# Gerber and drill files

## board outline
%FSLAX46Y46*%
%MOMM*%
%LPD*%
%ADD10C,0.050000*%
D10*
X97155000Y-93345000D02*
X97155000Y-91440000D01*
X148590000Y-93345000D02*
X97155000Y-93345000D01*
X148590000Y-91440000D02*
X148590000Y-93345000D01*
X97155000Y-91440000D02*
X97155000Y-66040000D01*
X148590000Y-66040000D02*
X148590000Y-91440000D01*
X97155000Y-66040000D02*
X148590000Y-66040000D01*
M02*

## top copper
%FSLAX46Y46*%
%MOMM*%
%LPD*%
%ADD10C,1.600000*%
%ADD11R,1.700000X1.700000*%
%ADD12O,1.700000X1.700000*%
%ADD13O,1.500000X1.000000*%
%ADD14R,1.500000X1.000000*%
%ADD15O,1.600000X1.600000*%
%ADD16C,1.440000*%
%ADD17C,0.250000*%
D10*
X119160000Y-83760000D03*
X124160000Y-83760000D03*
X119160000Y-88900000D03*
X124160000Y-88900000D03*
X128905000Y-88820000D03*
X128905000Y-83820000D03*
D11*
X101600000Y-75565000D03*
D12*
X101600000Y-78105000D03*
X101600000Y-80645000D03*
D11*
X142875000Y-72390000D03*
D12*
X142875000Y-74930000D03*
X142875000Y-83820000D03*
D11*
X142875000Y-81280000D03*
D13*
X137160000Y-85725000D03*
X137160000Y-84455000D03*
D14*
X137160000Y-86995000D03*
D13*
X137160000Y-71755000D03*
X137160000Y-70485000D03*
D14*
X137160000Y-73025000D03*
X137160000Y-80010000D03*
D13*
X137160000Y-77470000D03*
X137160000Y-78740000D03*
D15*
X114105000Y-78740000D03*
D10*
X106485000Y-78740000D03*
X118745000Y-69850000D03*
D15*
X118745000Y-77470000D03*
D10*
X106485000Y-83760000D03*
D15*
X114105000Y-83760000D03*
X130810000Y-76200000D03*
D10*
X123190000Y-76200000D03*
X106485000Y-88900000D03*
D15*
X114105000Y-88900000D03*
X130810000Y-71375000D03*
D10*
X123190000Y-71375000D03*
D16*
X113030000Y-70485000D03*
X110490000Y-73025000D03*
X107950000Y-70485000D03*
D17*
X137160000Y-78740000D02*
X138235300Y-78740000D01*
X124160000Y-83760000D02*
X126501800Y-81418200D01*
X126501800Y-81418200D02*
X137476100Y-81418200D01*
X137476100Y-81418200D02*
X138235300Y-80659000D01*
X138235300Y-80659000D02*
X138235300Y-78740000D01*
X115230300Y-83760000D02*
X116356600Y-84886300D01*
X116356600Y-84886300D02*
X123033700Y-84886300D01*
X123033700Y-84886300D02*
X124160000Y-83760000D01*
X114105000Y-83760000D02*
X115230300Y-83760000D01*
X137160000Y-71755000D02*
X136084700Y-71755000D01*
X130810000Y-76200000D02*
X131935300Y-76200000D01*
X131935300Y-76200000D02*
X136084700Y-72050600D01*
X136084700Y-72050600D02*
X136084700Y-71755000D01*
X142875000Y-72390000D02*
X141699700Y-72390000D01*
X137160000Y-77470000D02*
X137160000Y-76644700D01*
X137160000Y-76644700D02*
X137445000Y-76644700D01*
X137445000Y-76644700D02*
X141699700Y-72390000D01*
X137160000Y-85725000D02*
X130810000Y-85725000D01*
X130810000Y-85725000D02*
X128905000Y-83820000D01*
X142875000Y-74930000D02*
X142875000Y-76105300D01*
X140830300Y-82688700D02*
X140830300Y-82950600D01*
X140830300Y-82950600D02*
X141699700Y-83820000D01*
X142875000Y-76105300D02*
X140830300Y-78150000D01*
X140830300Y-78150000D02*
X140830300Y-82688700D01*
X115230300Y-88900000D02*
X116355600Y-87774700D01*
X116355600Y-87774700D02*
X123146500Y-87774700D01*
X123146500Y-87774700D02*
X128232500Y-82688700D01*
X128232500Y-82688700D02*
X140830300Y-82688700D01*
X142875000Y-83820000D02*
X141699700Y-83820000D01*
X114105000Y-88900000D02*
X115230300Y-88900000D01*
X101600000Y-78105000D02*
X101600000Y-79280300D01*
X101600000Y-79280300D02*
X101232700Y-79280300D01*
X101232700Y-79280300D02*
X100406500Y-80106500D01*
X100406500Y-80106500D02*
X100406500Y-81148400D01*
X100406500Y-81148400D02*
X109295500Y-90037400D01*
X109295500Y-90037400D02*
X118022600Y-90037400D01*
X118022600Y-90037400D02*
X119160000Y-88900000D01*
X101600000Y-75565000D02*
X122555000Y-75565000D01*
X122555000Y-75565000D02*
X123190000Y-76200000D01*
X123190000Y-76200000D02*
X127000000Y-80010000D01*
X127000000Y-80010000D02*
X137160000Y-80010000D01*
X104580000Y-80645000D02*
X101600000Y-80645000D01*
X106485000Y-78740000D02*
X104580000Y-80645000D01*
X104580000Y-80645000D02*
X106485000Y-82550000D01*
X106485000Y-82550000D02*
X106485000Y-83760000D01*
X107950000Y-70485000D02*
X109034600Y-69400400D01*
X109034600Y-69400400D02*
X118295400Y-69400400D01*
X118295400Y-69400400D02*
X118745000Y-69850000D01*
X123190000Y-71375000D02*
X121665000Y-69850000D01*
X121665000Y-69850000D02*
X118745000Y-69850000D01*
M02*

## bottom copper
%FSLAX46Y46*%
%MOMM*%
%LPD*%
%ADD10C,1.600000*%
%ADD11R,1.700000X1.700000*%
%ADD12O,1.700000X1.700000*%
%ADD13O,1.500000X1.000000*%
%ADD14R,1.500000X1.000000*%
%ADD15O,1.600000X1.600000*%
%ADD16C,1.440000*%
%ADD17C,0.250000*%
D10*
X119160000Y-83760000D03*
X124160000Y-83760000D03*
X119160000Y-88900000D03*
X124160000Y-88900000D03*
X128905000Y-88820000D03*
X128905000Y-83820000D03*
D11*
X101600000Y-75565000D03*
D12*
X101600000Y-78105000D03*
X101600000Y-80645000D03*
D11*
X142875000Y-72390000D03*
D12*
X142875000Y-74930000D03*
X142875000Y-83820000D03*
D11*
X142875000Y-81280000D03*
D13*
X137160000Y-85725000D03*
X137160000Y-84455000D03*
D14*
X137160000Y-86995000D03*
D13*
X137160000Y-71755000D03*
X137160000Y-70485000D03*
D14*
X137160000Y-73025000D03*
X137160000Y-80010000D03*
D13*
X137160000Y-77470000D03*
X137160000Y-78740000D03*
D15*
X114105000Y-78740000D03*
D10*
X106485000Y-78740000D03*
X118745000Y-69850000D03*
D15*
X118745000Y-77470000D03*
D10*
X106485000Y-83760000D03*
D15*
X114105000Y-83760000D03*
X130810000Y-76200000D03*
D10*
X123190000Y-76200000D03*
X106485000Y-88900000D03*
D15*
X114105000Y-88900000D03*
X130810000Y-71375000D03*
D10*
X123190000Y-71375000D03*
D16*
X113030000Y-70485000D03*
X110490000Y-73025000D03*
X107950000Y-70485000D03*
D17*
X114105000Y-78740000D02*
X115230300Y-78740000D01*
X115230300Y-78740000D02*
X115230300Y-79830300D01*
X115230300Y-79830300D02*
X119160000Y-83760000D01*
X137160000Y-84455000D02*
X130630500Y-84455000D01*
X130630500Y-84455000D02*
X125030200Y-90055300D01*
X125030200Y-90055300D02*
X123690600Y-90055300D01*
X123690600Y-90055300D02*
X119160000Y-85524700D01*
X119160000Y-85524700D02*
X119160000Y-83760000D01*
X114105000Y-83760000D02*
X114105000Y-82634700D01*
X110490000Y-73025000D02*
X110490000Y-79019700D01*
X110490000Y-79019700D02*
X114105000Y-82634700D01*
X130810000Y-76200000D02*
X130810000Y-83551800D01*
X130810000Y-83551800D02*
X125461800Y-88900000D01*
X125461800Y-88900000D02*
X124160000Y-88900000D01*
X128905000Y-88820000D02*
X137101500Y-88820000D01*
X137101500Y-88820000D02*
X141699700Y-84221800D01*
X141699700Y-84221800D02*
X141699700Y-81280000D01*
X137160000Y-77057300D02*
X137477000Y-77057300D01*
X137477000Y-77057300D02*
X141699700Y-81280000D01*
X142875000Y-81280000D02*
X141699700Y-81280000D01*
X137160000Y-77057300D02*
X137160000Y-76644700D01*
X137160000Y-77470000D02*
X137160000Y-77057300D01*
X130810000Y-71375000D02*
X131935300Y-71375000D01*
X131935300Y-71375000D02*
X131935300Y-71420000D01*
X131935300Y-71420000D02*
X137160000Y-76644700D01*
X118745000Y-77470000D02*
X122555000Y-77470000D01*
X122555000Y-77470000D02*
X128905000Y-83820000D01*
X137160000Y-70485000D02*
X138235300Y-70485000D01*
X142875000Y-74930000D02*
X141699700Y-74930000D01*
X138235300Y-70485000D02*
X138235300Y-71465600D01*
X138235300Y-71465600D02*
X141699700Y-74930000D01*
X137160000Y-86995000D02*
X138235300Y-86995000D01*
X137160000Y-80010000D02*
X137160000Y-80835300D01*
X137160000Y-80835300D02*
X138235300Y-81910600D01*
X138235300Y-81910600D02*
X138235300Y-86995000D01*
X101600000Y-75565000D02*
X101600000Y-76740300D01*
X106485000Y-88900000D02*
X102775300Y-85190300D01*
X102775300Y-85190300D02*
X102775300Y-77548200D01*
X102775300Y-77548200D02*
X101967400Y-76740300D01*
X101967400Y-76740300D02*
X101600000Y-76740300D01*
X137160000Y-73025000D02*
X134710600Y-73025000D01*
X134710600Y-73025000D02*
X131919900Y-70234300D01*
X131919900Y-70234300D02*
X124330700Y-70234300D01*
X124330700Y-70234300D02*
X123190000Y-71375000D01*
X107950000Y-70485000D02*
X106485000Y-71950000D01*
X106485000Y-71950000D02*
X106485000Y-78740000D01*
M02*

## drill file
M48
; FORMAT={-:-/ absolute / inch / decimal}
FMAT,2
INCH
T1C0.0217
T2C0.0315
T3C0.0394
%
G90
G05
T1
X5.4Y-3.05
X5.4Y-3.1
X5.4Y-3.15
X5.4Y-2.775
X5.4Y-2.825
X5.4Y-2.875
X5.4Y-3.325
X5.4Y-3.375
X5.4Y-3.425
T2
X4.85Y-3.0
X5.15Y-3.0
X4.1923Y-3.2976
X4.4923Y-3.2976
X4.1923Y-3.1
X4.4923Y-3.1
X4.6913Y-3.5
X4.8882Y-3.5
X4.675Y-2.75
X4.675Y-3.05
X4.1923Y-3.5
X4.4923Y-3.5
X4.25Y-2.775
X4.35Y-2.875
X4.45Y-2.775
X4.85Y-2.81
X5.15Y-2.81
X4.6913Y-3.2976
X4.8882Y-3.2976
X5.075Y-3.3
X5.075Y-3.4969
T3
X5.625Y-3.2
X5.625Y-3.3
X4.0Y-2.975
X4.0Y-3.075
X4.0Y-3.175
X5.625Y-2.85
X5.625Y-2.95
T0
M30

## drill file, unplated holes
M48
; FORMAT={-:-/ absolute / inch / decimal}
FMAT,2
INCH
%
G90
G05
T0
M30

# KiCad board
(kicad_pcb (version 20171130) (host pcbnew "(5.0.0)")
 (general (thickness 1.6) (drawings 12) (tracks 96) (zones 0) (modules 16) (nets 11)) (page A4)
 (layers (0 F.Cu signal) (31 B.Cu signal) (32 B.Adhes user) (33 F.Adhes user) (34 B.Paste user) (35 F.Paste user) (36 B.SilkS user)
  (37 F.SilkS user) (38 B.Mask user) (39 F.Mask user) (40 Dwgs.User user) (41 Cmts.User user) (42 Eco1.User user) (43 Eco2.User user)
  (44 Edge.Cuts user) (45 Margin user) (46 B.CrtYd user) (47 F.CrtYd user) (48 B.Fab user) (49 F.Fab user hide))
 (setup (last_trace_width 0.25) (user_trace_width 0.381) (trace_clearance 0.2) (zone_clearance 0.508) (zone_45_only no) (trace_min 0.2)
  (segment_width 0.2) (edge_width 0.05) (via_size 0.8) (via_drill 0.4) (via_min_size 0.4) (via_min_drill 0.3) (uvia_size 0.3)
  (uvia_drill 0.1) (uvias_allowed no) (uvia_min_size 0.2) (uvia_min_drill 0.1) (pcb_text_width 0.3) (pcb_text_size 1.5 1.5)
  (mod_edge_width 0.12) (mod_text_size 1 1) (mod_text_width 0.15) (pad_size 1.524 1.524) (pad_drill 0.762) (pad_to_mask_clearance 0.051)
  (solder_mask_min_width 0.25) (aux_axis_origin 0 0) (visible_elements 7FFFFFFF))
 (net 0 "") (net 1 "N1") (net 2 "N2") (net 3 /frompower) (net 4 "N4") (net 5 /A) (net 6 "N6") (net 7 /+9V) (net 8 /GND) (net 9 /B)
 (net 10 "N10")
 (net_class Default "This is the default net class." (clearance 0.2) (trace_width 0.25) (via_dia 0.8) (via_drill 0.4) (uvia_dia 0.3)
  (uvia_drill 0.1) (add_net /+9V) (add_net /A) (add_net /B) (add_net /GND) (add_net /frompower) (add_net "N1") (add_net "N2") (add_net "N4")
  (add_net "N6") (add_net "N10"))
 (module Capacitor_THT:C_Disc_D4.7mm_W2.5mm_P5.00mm (layer F.Cu) (at 119.16 83.76)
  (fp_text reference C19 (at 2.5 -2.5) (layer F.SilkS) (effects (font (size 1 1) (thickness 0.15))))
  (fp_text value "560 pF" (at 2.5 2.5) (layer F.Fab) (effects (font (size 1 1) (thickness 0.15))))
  (pad 1 thru_hole circle (at 0 0) (size 1.6 1.6) (drill 0.8) (layers *.Cu *.Mask) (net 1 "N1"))
  (pad 2 thru_hole circle (at 5 0) (size 1.6 1.6) (drill 0.8) (layers *.Cu *.Mask) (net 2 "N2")))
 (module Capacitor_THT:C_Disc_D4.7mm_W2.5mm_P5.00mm (layer F.Cu) (at 119.16 88.9)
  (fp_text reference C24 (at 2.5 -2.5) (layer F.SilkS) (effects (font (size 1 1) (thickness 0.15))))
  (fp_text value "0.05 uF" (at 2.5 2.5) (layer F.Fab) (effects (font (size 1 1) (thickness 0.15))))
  (pad 1 thru_hole circle (at 0 0) (size 1.6 1.6) (drill 0.8) (layers *.Cu *.Mask) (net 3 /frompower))
  (pad 2 thru_hole circle (at 5 0) (size 1.6 1.6) (drill 0.8) (layers *.Cu *.Mask) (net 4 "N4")))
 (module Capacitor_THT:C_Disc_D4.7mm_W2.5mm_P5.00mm (layer F.Cu) (at 128.905 83.82 270)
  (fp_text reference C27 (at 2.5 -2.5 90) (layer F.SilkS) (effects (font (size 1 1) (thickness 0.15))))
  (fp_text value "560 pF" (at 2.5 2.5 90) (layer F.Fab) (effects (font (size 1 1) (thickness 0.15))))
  (pad 2 thru_hole circle (at 5 0 270) (size 1.6 1.6) (drill 0.8) (layers *.Cu *.Mask) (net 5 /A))
  (pad 1 thru_hole circle (at 0 0 270) (size 1.6 1.6) (drill 0.8) (layers *.Cu *.Mask) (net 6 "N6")))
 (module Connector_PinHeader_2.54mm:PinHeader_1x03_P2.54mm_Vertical (layer F.Cu) (at 101.6 75.565)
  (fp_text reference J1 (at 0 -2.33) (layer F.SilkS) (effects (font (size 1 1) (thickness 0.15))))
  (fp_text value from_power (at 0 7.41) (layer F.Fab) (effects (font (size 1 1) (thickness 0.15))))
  (pad 1 thru_hole rect (at 0 0) (size 1.7 1.7) (drill 1) (layers *.Cu *.Mask) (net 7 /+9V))
  (pad 2 thru_hole oval (at 0 2.54) (size 1.7 1.7) (drill 1) (layers *.Cu *.Mask) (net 3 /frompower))
  (pad 3 thru_hole oval (at 0 5.08) (size 1.7 1.7) (drill 1) (layers *.Cu *.Mask) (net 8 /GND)))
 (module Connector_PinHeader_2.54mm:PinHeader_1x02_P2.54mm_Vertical (layer F.Cu) (at 142.875 72.39)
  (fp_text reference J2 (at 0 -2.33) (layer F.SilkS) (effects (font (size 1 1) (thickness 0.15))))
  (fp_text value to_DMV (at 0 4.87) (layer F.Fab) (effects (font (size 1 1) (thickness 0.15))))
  (pad 1 thru_hole rect (at 0 0) (size 1.7 1.7) (drill 1) (layers *.Cu *.Mask) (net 5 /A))
  (pad 2 thru_hole oval (at 0 2.54) (size 1.7 1.7) (drill 1) (layers *.Cu *.Mask) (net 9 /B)))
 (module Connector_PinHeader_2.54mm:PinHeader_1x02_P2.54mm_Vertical (layer F.Cu) (at 142.875 81.28)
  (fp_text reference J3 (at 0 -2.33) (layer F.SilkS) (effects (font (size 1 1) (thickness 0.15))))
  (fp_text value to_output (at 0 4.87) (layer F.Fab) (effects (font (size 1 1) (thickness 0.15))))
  (pad 2 thru_hole oval (at 0 2.54) (size 1.7 1.7) (drill 1) (layers *.Cu *.Mask) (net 9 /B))
  (pad 1 thru_hole rect (at 0 0) (size 1.7 1.7) (drill 1) (layers *.Cu *.Mask) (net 5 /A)))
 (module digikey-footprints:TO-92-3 (layer F.Cu) (at 137.16 86.995 90)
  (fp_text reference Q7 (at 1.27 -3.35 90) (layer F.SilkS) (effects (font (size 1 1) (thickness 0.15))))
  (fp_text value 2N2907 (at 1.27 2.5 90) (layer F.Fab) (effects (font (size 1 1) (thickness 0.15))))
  (pad 2 thru_hole oval (at 1.27 0 270) (size 1 1.5) (drill 0.55) (layers *.Cu *.Mask) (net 6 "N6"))
  (pad 3 thru_hole oval (at 2.54 0 270) (size 1 1.5) (drill 0.55) (layers *.Cu *.Mask) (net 1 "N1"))
  (pad 1 thru_hole rect (at 0 0 270) (size 1 1.5) (drill 0.55) (layers *.Cu *.Mask) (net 7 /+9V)))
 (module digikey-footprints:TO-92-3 (layer F.Cu) (at 137.16 73.025 90)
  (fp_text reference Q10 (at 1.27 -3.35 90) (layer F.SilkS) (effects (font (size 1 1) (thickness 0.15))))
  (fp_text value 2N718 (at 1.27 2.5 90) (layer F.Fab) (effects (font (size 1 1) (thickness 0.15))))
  (pad 2 thru_hole oval (at 1.27 0 270) (size 1 1.5) (drill 0.55) (layers *.Cu *.Mask) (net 4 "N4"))
  (pad 3 thru_hole oval (at 2.54 0 270) (size 1 1.5) (drill 0.55) (layers *.Cu *.Mask) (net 9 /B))
  (pad 1 thru_hole rect (at 0 0 270) (size 1 1.5) (drill 0.55) (layers *.Cu *.Mask) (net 8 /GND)))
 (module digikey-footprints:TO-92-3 (layer F.Cu) (at 137.16 80.01 90)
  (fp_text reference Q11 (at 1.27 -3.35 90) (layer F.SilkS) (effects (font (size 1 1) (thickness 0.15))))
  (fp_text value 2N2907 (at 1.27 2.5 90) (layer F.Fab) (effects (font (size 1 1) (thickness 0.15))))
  (pad 1 thru_hole rect (at 0 0 270) (size 1 1.5) (drill 0.55) (layers *.Cu *.Mask) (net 7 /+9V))
  (pad 3 thru_hole oval (at 2.54 0 270) (size 1 1.5) (drill 0.55) (layers *.Cu *.Mask) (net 5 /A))
  (pad 2 thru_hole oval (at 1.27 0 270) (size 1 1.5) (drill 0.55) (layers *.Cu *.Mask) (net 2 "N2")))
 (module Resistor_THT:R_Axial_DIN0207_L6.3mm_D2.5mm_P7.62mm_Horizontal (layer F.Cu) (at 106.485 78.74)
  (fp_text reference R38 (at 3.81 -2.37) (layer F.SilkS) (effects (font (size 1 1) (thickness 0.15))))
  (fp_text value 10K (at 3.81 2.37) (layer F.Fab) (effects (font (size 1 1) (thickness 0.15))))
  (pad 2 thru_hole oval (at 7.62 0) (size 1.6 1.6) (drill 0.8) (layers *.Cu *.Mask) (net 1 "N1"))
  (pad 1 thru_hole circle (at 0 0) (size 1.6 1.6) (drill 0.8) (layers *.Cu *.Mask) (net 8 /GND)))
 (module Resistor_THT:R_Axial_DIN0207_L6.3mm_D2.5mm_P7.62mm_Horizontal (layer F.Cu) (at 118.745 69.85 270)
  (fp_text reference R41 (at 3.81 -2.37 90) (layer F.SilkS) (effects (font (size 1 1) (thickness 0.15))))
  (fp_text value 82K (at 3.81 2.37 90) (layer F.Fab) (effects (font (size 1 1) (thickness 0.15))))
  (pad 1 thru_hole circle (at 0 0 270) (size 1.6 1.6) (drill 0.8) (layers *.Cu *.Mask) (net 8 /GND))
  (pad 2 thru_hole oval (at 7.62 0 270) (size 1.6 1.6) (drill 0.8) (layers *.Cu *.Mask) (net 6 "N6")))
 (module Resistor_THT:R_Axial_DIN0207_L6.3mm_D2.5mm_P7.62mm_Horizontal (layer F.Cu) (at 106.485 83.76)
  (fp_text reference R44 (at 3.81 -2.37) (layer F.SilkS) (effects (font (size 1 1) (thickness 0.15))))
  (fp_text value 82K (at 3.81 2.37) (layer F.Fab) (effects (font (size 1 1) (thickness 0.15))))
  (pad 1 thru_hole circle (at 0 0) (size 1.6 1.6) (drill 0.8) (layers *.Cu *.Mask) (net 8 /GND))
  (pad 2 thru_hole oval (at 7.62 0) (size 1.6 1.6) (drill 0.8) (layers *.Cu *.Mask) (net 2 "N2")))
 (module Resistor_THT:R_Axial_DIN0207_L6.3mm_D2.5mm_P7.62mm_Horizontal (layer F.Cu) (at 123.19 76.2)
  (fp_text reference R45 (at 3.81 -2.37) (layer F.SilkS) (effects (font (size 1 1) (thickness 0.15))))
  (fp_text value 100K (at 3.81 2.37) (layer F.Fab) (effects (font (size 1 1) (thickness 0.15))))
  (pad 2 thru_hole oval (at 7.62 0) (size 1.6 1.6) (drill 0.8) (layers *.Cu *.Mask) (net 4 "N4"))
  (pad 1 thru_hole circle (at 0 0) (size 1.6 1.6) (drill 0.8) (layers *.Cu *.Mask) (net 7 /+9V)))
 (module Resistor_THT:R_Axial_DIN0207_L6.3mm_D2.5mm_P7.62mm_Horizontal (layer F.Cu) (at 106.485 88.9)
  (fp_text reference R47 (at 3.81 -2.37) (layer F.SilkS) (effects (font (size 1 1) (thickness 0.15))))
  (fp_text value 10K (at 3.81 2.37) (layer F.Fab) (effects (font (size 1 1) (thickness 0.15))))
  (pad 1 thru_hole circle (at 0 0) (size 1.6 1.6) (drill 0.8) (layers *.Cu *.Mask) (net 7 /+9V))
  (pad 2 thru_hole oval (at 7.62 0) (size 1.6 1.6) (drill 0.8) (layers *.Cu *.Mask) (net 9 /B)))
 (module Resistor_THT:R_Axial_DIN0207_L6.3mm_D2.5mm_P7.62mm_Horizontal (layer F.Cu) (at 123.19 71.375)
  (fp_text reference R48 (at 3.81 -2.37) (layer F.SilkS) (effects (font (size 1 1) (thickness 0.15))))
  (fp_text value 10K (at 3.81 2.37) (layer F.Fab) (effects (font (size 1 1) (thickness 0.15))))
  (pad 2 thru_hole oval (at 7.62 0) (size 1.6 1.6) (drill 0.8) (layers *.Cu *.Mask) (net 5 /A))
  (pad 1 thru_hole circle (at 0 0) (size 1.6 1.6) (drill 0.8) (layers *.Cu *.Mask) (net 8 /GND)))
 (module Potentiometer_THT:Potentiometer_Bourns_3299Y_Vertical (layer F.Cu) (at 113.03 70.485)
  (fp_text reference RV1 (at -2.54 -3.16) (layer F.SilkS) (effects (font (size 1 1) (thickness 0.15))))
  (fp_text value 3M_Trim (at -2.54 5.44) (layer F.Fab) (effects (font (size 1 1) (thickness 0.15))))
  (pad 1 thru_hole circle (at 0 0) (size 1.44 1.44) (drill 0.8) (layers *.Cu *.Mask) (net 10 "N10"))
  (pad 2 thru_hole circle (at -2.54 2.54) (size 1.44 1.44) (drill 0.8) (layers *.Cu *.Mask) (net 2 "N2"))
  (pad 3 thru_hole circle (at -5.08 0) (size 1.44 1.44) (drill 0.8) (layers *.Cu *.Mask) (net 8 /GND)))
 (gr_line (start 97.155 93.345) (end 97.155 91.44) (layer Edge.Cuts) (width 0.05))
 (gr_line (start 148.59 93.345) (end 97.155 93.345) (layer Edge.Cuts) (width 0.05))
 (gr_line (start 148.59 91.44) (end 148.59 93.345) (layer Edge.Cuts) (width 0.05))
 (gr_line (start 97.155 91.44) (end 97.155 66.04) (layer Edge.Cuts) (width 0.05))
 (gr_line (start 148.59 66.04) (end 148.59 91.44) (layer Edge.Cuts) (width 0.05))
 (gr_line (start 97.155 66.04) (end 148.59 66.04) (layer Edge.Cuts) (width 0.05))
 (segment (start 114.105 78.74) (end 115.2303 78.74) (width 0.25) (layer B.Cu) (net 1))
 (segment (start 115.2303 78.74) (end 115.2303 79.8303) (width 0.25) (layer B.Cu) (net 1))
 (segment (start 115.2303 79.8303) (end 119.16 83.76) (width 0.25) (layer B.Cu) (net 1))
 (segment (start 137.16 84.455) (end 130.6305 84.455) (width 0.25) (layer B.Cu) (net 1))
 (segment (start 130.6305 84.455) (end 125.0302 90.0553) (width 0.25) (layer B.Cu) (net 1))
 (segment (start 125.0302 90.0553) (end 123.6906 90.0553) (width 0.25) (layer B.Cu) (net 1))
 (segment (start 123.6906 90.0553) (end 119.16 85.5247) (width 0.25) (layer B.Cu) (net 1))
 (segment (start 119.16 85.5247) (end 119.16 83.76) (width 0.25) (layer B.Cu) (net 1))
 (segment (start 137.16 78.74) (end 138.2353 78.74) (width 0.25) (layer F.Cu) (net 2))
 (segment (start 124.16 83.76) (end 126.5018 81.4182) (width 0.25) (layer F.Cu) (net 2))
 (segment (start 126.5018 81.4182) (end 137.4761 81.4182) (width 0.25) (layer F.Cu) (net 2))
 (segment (start 137.4761 81.4182) (end 138.2353 80.659) (width 0.25) (layer F.Cu) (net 2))
 (segment (start 138.2353 80.659) (end 138.2353 78.74) (width 0.25) (layer F.Cu) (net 2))
 (segment (start 115.2303 83.76) (end 116.3566 84.8863) (width 0.25) (layer F.Cu) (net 2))
 (segment (start 116.3566 84.8863) (end 123.0337 84.8863) (width 0.25) (layer F.Cu) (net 2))
 (segment (start 123.0337 84.8863) (end 124.16 83.76) (width 0.25) (layer F.Cu) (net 2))
 (segment (start 114.105 83.76) (end 115.2303 83.76) (width 0.25) (layer F.Cu) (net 2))
 (segment (start 114.105 83.76) (end 114.105 82.6347) (width 0.25) (layer B.Cu) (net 2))
 (segment (start 110.49 73.025) (end 110.49 79.0197) (width 0.25) (layer B.Cu) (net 2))
 (segment (start 110.49 79.0197) (end 114.105 82.6347) (width 0.25) (layer B.Cu) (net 2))
 (segment (start 130.81 76.2) (end 130.81 83.5518) (width 0.25) (layer B.Cu) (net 4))
 (segment (start 130.81 83.5518) (end 125.4618 88.9) (width 0.25) (layer B.Cu) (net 4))
 (segment (start 125.4618 88.9) (end 124.16 88.9) (width 0.25) (layer B.Cu) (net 4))
 (segment (start 137.16 71.755) (end 136.0847 71.755) (width 0.25) (layer F.Cu) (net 4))
 (segment (start 130.81 76.2) (end 131.9353 76.2) (width 0.25) (layer F.Cu) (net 4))
 (segment (start 131.9353 76.2) (end 136.0847 72.0506) (width 0.25) (layer F.Cu) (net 4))
 (segment (start 136.0847 72.0506) (end 136.0847 71.755) (width 0.25) (layer F.Cu) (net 4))
 (segment (start 142.875 72.39) (end 141.6997 72.39) (width 0.25) (layer F.Cu) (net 5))
 (segment (start 137.16 77.47) (end 137.16 76.6447) (width 0.25) (layer F.Cu) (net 5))
 (segment (start 137.16 76.6447) (end 137.445 76.6447) (width 0.25) (layer F.Cu) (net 5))
 (segment (start 137.445 76.6447) (end 141.6997 72.39) (width 0.25) (layer F.Cu) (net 5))
 (segment (start 128.905 88.82) (end 137.1015 88.82) (width 0.25) (layer B.Cu) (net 5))
 (segment (start 137.1015 88.82) (end 141.6997 84.2218) (width 0.25) (layer B.Cu) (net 5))
 (segment (start 141.6997 84.2218) (end 141.6997 81.28) (width 0.25) (layer B.Cu) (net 5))
 (segment (start 137.16 77.0573) (end 137.477 77.0573) (width 0.25) (layer B.Cu) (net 5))
 (segment (start 137.477 77.0573) (end 141.6997 81.28) (width 0.25) (layer B.Cu) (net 5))
 (segment (start 142.875 81.28) (end 141.6997 81.28) (width 0.25) (layer B.Cu) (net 5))
 (segment (start 137.16 77.0573) (end 137.16 76.6447) (width 0.25) (layer B.Cu) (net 5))
 (segment (start 137.16 77.47) (end 137.16 77.0573) (width 0.25) (layer B.Cu) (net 5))
 (segment (start 130.81 71.375) (end 131.9353 71.375) (width 0.25) (layer B.Cu) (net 5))
 (segment (start 131.9353 71.375) (end 131.9353 71.42) (width 0.25) (layer B.Cu) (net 5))
 (segment (start 131.9353 71.42) (end 137.16 76.6447) (width 0.25) (layer B.Cu) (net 5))
 (segment (start 137.16 85.725) (end 130.81 85.725) (width 0.25) (layer F.Cu) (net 6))
 (segment (start 130.81 85.725) (end 128.905 83.82) (width 0.25) (layer F.Cu) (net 6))
 (segment (start 118.745 77.47) (end 122.555 77.47) (width 0.25) (layer B.Cu) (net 6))
 (segment (start 122.555 77.47) (end 128.905 83.82) (width 0.25) (layer B.Cu) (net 6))
 (segment (start 142.875 74.93) (end 142.875 76.1053) (width 0.25) (layer F.Cu) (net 9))
 (segment (start 140.8303 82.6887) (end 140.8303 82.9506) (width 0.25) (layer F.Cu) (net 9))
 (segment (start 140.8303 82.9506) (end 141.6997 83.82) (width 0.25) (layer F.Cu) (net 9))
 (segment (start 142.875 76.1053) (end 140.8303 78.15) (width 0.25) (layer F.Cu) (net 9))
 (segment (start 140.8303 78.15) (end 140.8303 82.6887) (width 0.25) (layer F.Cu) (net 9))
 (segment (start 115.2303 88.9) (end 116.3556 87.7747) (width 0.25) (layer F.Cu) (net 9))
 (segment (start 116.3556 87.7747) (end 123.1465 87.7747) (width 0.25) (layer F.Cu) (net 9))
 (segment (start 123.1465 87.7747) (end 128.2325 82.6887) (width 0.25) (layer F.Cu) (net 9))
 (segment (start 128.2325 82.6887) (end 140.8303 82.6887) (width 0.25) (layer F.Cu) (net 9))
 (segment (start 142.875 83.82) (end 141.6997 83.82) (width 0.25) (layer F.Cu) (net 9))
 (segment (start 114.105 88.9) (end 115.2303 88.9) (width 0.25) (layer F.Cu) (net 9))
 (segment (start 137.16 70.485) (end 138.2353 70.485) (width 0.25) (layer B.Cu) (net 9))
 (segment (start 142.875 74.93) (end 141.6997 74.93) (width 0.25) (layer B.Cu) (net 9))
 (segment (start 138.2353 70.485) (end 138.2353 71.4656) (width 0.25) (layer B.Cu) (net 9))
 (segment (start 138.2353 71.4656) (end 141.6997 74.93) (width 0.25) (layer B.Cu) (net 9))
 (segment (start 101.6 78.105) (end 101.6 79.2803) (width 0.25) (layer F.Cu) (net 3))
 (segment (start 101.6 79.2803) (end 101.2327 79.2803) (width 0.25) (layer F.Cu) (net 3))
 (segment (start 101.2327 79.2803) (end 100.4065 80.1065) (width 0.25) (layer F.Cu) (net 3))
 (segment (start 100.4065 80.1065) (end 100.4065 81.1484) (width 0.25) (layer F.Cu) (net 3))
 (segment (start 100.4065 81.1484) (end 109.2955 90.0374) (width 0.25) (layer F.Cu) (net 3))
 (segment (start 109.2955 90.0374) (end 118.0226 90.0374) (width 0.25) (layer F.Cu) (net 3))
 (segment (start 118.0226 90.0374) (end 119.16 88.9) (width 0.25) (layer F.Cu) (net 3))
 (segment (start 101.6 75.565) (end 122.555 75.565) (width 0.25) (layer F.Cu) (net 7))
 (segment (start 122.555 75.565) (end 123.19 76.2) (width 0.25) (layer F.Cu) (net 7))
 (segment (start 123.19 76.2) (end 127 80.01) (width 0.25) (layer F.Cu) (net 7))
 (segment (start 127 80.01) (end 137.16 80.01) (width 0.25) (layer F.Cu) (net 7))
 (segment (start 137.16 86.995) (end 138.2353 86.995) (width 0.25) (layer B.Cu) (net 7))
 (segment (start 137.16 80.01) (end 137.16 80.8353) (width 0.25) (layer B.Cu) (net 7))
 (segment (start 137.16 80.8353) (end 138.2353 81.9106) (width 0.25) (layer B.Cu) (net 7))
 (segment (start 138.2353 81.9106) (end 138.2353 86.995) (width 0.25) (layer B.Cu) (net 7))
 (segment (start 101.6 75.565) (end 101.6 76.7403) (width 0.25) (layer B.Cu) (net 7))
 (segment (start 106.485 88.9) (end 102.7753 85.1903) (width 0.25) (layer B.Cu) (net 7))
 (segment (start 102.7753 85.1903) (end 102.7753 77.5482) (width 0.25) (layer B.Cu) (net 7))
 (segment (start 102.7753 77.5482) (end 101.9674 76.7403) (width 0.25) (layer B.Cu) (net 7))
 (segment (start 101.9674 76.7403) (end 101.6 76.7403) (width 0.25) (layer B.Cu) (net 7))
 (segment (start 104.58 80.645) (end 101.6 80.645) (width 0.25) (layer F.Cu) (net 8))
 (segment (start 106.485 78.74) (end 104.58 80.645) (width 0.25) (layer F.Cu) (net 8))
 (segment (start 104.58 80.645) (end 106.485 82.55) (width 0.25) (layer F.Cu) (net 8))
 (segment (start 106.485 82.55) (end 106.485 83.76) (width 0.25) (layer F.Cu) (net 8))
 (segment (start 107.95 70.485) (end 109.0346 69.4004) (width 0.25) (layer F.Cu) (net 8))
 (segment (start 109.0346 69.4004) (end 118.2954 69.4004) (width 0.25) (layer F.Cu) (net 8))
 (segment (start 118.2954 69.4004) (end 118.745 69.85) (width 0.25) (layer F.Cu) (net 8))
 (segment (start 137.16 73.025) (end 134.7106 73.025) (width 0.25) (layer B.Cu) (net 8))
 (segment (start 134.7106 73.025) (end 131.9199 70.2343) (width 0.25) (layer B.Cu) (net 8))
 (segment (start 131.9199 70.2343) (end 124.3307 70.2343) (width 0.25) (layer B.Cu) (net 8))
 (segment (start 124.3307 70.2343) (end 123.19 71.375) (width 0.25) (layer B.Cu) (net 8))
 (segment (start 123.19 71.375) (end 121.665 69.85) (width 0.25) (layer F.Cu) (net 8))
 (segment (start 121.665 69.85) (end 118.745 69.85) (width 0.25) (layer F.Cu) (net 8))
 (segment (start 107.95 70.485) (end 106.485 71.95) (width 0.25) (layer B.Cu) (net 8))
 (segment (start 106.485 71.95) (end 106.485 78.74) (width 0.25) (layer B.Cu) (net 8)))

